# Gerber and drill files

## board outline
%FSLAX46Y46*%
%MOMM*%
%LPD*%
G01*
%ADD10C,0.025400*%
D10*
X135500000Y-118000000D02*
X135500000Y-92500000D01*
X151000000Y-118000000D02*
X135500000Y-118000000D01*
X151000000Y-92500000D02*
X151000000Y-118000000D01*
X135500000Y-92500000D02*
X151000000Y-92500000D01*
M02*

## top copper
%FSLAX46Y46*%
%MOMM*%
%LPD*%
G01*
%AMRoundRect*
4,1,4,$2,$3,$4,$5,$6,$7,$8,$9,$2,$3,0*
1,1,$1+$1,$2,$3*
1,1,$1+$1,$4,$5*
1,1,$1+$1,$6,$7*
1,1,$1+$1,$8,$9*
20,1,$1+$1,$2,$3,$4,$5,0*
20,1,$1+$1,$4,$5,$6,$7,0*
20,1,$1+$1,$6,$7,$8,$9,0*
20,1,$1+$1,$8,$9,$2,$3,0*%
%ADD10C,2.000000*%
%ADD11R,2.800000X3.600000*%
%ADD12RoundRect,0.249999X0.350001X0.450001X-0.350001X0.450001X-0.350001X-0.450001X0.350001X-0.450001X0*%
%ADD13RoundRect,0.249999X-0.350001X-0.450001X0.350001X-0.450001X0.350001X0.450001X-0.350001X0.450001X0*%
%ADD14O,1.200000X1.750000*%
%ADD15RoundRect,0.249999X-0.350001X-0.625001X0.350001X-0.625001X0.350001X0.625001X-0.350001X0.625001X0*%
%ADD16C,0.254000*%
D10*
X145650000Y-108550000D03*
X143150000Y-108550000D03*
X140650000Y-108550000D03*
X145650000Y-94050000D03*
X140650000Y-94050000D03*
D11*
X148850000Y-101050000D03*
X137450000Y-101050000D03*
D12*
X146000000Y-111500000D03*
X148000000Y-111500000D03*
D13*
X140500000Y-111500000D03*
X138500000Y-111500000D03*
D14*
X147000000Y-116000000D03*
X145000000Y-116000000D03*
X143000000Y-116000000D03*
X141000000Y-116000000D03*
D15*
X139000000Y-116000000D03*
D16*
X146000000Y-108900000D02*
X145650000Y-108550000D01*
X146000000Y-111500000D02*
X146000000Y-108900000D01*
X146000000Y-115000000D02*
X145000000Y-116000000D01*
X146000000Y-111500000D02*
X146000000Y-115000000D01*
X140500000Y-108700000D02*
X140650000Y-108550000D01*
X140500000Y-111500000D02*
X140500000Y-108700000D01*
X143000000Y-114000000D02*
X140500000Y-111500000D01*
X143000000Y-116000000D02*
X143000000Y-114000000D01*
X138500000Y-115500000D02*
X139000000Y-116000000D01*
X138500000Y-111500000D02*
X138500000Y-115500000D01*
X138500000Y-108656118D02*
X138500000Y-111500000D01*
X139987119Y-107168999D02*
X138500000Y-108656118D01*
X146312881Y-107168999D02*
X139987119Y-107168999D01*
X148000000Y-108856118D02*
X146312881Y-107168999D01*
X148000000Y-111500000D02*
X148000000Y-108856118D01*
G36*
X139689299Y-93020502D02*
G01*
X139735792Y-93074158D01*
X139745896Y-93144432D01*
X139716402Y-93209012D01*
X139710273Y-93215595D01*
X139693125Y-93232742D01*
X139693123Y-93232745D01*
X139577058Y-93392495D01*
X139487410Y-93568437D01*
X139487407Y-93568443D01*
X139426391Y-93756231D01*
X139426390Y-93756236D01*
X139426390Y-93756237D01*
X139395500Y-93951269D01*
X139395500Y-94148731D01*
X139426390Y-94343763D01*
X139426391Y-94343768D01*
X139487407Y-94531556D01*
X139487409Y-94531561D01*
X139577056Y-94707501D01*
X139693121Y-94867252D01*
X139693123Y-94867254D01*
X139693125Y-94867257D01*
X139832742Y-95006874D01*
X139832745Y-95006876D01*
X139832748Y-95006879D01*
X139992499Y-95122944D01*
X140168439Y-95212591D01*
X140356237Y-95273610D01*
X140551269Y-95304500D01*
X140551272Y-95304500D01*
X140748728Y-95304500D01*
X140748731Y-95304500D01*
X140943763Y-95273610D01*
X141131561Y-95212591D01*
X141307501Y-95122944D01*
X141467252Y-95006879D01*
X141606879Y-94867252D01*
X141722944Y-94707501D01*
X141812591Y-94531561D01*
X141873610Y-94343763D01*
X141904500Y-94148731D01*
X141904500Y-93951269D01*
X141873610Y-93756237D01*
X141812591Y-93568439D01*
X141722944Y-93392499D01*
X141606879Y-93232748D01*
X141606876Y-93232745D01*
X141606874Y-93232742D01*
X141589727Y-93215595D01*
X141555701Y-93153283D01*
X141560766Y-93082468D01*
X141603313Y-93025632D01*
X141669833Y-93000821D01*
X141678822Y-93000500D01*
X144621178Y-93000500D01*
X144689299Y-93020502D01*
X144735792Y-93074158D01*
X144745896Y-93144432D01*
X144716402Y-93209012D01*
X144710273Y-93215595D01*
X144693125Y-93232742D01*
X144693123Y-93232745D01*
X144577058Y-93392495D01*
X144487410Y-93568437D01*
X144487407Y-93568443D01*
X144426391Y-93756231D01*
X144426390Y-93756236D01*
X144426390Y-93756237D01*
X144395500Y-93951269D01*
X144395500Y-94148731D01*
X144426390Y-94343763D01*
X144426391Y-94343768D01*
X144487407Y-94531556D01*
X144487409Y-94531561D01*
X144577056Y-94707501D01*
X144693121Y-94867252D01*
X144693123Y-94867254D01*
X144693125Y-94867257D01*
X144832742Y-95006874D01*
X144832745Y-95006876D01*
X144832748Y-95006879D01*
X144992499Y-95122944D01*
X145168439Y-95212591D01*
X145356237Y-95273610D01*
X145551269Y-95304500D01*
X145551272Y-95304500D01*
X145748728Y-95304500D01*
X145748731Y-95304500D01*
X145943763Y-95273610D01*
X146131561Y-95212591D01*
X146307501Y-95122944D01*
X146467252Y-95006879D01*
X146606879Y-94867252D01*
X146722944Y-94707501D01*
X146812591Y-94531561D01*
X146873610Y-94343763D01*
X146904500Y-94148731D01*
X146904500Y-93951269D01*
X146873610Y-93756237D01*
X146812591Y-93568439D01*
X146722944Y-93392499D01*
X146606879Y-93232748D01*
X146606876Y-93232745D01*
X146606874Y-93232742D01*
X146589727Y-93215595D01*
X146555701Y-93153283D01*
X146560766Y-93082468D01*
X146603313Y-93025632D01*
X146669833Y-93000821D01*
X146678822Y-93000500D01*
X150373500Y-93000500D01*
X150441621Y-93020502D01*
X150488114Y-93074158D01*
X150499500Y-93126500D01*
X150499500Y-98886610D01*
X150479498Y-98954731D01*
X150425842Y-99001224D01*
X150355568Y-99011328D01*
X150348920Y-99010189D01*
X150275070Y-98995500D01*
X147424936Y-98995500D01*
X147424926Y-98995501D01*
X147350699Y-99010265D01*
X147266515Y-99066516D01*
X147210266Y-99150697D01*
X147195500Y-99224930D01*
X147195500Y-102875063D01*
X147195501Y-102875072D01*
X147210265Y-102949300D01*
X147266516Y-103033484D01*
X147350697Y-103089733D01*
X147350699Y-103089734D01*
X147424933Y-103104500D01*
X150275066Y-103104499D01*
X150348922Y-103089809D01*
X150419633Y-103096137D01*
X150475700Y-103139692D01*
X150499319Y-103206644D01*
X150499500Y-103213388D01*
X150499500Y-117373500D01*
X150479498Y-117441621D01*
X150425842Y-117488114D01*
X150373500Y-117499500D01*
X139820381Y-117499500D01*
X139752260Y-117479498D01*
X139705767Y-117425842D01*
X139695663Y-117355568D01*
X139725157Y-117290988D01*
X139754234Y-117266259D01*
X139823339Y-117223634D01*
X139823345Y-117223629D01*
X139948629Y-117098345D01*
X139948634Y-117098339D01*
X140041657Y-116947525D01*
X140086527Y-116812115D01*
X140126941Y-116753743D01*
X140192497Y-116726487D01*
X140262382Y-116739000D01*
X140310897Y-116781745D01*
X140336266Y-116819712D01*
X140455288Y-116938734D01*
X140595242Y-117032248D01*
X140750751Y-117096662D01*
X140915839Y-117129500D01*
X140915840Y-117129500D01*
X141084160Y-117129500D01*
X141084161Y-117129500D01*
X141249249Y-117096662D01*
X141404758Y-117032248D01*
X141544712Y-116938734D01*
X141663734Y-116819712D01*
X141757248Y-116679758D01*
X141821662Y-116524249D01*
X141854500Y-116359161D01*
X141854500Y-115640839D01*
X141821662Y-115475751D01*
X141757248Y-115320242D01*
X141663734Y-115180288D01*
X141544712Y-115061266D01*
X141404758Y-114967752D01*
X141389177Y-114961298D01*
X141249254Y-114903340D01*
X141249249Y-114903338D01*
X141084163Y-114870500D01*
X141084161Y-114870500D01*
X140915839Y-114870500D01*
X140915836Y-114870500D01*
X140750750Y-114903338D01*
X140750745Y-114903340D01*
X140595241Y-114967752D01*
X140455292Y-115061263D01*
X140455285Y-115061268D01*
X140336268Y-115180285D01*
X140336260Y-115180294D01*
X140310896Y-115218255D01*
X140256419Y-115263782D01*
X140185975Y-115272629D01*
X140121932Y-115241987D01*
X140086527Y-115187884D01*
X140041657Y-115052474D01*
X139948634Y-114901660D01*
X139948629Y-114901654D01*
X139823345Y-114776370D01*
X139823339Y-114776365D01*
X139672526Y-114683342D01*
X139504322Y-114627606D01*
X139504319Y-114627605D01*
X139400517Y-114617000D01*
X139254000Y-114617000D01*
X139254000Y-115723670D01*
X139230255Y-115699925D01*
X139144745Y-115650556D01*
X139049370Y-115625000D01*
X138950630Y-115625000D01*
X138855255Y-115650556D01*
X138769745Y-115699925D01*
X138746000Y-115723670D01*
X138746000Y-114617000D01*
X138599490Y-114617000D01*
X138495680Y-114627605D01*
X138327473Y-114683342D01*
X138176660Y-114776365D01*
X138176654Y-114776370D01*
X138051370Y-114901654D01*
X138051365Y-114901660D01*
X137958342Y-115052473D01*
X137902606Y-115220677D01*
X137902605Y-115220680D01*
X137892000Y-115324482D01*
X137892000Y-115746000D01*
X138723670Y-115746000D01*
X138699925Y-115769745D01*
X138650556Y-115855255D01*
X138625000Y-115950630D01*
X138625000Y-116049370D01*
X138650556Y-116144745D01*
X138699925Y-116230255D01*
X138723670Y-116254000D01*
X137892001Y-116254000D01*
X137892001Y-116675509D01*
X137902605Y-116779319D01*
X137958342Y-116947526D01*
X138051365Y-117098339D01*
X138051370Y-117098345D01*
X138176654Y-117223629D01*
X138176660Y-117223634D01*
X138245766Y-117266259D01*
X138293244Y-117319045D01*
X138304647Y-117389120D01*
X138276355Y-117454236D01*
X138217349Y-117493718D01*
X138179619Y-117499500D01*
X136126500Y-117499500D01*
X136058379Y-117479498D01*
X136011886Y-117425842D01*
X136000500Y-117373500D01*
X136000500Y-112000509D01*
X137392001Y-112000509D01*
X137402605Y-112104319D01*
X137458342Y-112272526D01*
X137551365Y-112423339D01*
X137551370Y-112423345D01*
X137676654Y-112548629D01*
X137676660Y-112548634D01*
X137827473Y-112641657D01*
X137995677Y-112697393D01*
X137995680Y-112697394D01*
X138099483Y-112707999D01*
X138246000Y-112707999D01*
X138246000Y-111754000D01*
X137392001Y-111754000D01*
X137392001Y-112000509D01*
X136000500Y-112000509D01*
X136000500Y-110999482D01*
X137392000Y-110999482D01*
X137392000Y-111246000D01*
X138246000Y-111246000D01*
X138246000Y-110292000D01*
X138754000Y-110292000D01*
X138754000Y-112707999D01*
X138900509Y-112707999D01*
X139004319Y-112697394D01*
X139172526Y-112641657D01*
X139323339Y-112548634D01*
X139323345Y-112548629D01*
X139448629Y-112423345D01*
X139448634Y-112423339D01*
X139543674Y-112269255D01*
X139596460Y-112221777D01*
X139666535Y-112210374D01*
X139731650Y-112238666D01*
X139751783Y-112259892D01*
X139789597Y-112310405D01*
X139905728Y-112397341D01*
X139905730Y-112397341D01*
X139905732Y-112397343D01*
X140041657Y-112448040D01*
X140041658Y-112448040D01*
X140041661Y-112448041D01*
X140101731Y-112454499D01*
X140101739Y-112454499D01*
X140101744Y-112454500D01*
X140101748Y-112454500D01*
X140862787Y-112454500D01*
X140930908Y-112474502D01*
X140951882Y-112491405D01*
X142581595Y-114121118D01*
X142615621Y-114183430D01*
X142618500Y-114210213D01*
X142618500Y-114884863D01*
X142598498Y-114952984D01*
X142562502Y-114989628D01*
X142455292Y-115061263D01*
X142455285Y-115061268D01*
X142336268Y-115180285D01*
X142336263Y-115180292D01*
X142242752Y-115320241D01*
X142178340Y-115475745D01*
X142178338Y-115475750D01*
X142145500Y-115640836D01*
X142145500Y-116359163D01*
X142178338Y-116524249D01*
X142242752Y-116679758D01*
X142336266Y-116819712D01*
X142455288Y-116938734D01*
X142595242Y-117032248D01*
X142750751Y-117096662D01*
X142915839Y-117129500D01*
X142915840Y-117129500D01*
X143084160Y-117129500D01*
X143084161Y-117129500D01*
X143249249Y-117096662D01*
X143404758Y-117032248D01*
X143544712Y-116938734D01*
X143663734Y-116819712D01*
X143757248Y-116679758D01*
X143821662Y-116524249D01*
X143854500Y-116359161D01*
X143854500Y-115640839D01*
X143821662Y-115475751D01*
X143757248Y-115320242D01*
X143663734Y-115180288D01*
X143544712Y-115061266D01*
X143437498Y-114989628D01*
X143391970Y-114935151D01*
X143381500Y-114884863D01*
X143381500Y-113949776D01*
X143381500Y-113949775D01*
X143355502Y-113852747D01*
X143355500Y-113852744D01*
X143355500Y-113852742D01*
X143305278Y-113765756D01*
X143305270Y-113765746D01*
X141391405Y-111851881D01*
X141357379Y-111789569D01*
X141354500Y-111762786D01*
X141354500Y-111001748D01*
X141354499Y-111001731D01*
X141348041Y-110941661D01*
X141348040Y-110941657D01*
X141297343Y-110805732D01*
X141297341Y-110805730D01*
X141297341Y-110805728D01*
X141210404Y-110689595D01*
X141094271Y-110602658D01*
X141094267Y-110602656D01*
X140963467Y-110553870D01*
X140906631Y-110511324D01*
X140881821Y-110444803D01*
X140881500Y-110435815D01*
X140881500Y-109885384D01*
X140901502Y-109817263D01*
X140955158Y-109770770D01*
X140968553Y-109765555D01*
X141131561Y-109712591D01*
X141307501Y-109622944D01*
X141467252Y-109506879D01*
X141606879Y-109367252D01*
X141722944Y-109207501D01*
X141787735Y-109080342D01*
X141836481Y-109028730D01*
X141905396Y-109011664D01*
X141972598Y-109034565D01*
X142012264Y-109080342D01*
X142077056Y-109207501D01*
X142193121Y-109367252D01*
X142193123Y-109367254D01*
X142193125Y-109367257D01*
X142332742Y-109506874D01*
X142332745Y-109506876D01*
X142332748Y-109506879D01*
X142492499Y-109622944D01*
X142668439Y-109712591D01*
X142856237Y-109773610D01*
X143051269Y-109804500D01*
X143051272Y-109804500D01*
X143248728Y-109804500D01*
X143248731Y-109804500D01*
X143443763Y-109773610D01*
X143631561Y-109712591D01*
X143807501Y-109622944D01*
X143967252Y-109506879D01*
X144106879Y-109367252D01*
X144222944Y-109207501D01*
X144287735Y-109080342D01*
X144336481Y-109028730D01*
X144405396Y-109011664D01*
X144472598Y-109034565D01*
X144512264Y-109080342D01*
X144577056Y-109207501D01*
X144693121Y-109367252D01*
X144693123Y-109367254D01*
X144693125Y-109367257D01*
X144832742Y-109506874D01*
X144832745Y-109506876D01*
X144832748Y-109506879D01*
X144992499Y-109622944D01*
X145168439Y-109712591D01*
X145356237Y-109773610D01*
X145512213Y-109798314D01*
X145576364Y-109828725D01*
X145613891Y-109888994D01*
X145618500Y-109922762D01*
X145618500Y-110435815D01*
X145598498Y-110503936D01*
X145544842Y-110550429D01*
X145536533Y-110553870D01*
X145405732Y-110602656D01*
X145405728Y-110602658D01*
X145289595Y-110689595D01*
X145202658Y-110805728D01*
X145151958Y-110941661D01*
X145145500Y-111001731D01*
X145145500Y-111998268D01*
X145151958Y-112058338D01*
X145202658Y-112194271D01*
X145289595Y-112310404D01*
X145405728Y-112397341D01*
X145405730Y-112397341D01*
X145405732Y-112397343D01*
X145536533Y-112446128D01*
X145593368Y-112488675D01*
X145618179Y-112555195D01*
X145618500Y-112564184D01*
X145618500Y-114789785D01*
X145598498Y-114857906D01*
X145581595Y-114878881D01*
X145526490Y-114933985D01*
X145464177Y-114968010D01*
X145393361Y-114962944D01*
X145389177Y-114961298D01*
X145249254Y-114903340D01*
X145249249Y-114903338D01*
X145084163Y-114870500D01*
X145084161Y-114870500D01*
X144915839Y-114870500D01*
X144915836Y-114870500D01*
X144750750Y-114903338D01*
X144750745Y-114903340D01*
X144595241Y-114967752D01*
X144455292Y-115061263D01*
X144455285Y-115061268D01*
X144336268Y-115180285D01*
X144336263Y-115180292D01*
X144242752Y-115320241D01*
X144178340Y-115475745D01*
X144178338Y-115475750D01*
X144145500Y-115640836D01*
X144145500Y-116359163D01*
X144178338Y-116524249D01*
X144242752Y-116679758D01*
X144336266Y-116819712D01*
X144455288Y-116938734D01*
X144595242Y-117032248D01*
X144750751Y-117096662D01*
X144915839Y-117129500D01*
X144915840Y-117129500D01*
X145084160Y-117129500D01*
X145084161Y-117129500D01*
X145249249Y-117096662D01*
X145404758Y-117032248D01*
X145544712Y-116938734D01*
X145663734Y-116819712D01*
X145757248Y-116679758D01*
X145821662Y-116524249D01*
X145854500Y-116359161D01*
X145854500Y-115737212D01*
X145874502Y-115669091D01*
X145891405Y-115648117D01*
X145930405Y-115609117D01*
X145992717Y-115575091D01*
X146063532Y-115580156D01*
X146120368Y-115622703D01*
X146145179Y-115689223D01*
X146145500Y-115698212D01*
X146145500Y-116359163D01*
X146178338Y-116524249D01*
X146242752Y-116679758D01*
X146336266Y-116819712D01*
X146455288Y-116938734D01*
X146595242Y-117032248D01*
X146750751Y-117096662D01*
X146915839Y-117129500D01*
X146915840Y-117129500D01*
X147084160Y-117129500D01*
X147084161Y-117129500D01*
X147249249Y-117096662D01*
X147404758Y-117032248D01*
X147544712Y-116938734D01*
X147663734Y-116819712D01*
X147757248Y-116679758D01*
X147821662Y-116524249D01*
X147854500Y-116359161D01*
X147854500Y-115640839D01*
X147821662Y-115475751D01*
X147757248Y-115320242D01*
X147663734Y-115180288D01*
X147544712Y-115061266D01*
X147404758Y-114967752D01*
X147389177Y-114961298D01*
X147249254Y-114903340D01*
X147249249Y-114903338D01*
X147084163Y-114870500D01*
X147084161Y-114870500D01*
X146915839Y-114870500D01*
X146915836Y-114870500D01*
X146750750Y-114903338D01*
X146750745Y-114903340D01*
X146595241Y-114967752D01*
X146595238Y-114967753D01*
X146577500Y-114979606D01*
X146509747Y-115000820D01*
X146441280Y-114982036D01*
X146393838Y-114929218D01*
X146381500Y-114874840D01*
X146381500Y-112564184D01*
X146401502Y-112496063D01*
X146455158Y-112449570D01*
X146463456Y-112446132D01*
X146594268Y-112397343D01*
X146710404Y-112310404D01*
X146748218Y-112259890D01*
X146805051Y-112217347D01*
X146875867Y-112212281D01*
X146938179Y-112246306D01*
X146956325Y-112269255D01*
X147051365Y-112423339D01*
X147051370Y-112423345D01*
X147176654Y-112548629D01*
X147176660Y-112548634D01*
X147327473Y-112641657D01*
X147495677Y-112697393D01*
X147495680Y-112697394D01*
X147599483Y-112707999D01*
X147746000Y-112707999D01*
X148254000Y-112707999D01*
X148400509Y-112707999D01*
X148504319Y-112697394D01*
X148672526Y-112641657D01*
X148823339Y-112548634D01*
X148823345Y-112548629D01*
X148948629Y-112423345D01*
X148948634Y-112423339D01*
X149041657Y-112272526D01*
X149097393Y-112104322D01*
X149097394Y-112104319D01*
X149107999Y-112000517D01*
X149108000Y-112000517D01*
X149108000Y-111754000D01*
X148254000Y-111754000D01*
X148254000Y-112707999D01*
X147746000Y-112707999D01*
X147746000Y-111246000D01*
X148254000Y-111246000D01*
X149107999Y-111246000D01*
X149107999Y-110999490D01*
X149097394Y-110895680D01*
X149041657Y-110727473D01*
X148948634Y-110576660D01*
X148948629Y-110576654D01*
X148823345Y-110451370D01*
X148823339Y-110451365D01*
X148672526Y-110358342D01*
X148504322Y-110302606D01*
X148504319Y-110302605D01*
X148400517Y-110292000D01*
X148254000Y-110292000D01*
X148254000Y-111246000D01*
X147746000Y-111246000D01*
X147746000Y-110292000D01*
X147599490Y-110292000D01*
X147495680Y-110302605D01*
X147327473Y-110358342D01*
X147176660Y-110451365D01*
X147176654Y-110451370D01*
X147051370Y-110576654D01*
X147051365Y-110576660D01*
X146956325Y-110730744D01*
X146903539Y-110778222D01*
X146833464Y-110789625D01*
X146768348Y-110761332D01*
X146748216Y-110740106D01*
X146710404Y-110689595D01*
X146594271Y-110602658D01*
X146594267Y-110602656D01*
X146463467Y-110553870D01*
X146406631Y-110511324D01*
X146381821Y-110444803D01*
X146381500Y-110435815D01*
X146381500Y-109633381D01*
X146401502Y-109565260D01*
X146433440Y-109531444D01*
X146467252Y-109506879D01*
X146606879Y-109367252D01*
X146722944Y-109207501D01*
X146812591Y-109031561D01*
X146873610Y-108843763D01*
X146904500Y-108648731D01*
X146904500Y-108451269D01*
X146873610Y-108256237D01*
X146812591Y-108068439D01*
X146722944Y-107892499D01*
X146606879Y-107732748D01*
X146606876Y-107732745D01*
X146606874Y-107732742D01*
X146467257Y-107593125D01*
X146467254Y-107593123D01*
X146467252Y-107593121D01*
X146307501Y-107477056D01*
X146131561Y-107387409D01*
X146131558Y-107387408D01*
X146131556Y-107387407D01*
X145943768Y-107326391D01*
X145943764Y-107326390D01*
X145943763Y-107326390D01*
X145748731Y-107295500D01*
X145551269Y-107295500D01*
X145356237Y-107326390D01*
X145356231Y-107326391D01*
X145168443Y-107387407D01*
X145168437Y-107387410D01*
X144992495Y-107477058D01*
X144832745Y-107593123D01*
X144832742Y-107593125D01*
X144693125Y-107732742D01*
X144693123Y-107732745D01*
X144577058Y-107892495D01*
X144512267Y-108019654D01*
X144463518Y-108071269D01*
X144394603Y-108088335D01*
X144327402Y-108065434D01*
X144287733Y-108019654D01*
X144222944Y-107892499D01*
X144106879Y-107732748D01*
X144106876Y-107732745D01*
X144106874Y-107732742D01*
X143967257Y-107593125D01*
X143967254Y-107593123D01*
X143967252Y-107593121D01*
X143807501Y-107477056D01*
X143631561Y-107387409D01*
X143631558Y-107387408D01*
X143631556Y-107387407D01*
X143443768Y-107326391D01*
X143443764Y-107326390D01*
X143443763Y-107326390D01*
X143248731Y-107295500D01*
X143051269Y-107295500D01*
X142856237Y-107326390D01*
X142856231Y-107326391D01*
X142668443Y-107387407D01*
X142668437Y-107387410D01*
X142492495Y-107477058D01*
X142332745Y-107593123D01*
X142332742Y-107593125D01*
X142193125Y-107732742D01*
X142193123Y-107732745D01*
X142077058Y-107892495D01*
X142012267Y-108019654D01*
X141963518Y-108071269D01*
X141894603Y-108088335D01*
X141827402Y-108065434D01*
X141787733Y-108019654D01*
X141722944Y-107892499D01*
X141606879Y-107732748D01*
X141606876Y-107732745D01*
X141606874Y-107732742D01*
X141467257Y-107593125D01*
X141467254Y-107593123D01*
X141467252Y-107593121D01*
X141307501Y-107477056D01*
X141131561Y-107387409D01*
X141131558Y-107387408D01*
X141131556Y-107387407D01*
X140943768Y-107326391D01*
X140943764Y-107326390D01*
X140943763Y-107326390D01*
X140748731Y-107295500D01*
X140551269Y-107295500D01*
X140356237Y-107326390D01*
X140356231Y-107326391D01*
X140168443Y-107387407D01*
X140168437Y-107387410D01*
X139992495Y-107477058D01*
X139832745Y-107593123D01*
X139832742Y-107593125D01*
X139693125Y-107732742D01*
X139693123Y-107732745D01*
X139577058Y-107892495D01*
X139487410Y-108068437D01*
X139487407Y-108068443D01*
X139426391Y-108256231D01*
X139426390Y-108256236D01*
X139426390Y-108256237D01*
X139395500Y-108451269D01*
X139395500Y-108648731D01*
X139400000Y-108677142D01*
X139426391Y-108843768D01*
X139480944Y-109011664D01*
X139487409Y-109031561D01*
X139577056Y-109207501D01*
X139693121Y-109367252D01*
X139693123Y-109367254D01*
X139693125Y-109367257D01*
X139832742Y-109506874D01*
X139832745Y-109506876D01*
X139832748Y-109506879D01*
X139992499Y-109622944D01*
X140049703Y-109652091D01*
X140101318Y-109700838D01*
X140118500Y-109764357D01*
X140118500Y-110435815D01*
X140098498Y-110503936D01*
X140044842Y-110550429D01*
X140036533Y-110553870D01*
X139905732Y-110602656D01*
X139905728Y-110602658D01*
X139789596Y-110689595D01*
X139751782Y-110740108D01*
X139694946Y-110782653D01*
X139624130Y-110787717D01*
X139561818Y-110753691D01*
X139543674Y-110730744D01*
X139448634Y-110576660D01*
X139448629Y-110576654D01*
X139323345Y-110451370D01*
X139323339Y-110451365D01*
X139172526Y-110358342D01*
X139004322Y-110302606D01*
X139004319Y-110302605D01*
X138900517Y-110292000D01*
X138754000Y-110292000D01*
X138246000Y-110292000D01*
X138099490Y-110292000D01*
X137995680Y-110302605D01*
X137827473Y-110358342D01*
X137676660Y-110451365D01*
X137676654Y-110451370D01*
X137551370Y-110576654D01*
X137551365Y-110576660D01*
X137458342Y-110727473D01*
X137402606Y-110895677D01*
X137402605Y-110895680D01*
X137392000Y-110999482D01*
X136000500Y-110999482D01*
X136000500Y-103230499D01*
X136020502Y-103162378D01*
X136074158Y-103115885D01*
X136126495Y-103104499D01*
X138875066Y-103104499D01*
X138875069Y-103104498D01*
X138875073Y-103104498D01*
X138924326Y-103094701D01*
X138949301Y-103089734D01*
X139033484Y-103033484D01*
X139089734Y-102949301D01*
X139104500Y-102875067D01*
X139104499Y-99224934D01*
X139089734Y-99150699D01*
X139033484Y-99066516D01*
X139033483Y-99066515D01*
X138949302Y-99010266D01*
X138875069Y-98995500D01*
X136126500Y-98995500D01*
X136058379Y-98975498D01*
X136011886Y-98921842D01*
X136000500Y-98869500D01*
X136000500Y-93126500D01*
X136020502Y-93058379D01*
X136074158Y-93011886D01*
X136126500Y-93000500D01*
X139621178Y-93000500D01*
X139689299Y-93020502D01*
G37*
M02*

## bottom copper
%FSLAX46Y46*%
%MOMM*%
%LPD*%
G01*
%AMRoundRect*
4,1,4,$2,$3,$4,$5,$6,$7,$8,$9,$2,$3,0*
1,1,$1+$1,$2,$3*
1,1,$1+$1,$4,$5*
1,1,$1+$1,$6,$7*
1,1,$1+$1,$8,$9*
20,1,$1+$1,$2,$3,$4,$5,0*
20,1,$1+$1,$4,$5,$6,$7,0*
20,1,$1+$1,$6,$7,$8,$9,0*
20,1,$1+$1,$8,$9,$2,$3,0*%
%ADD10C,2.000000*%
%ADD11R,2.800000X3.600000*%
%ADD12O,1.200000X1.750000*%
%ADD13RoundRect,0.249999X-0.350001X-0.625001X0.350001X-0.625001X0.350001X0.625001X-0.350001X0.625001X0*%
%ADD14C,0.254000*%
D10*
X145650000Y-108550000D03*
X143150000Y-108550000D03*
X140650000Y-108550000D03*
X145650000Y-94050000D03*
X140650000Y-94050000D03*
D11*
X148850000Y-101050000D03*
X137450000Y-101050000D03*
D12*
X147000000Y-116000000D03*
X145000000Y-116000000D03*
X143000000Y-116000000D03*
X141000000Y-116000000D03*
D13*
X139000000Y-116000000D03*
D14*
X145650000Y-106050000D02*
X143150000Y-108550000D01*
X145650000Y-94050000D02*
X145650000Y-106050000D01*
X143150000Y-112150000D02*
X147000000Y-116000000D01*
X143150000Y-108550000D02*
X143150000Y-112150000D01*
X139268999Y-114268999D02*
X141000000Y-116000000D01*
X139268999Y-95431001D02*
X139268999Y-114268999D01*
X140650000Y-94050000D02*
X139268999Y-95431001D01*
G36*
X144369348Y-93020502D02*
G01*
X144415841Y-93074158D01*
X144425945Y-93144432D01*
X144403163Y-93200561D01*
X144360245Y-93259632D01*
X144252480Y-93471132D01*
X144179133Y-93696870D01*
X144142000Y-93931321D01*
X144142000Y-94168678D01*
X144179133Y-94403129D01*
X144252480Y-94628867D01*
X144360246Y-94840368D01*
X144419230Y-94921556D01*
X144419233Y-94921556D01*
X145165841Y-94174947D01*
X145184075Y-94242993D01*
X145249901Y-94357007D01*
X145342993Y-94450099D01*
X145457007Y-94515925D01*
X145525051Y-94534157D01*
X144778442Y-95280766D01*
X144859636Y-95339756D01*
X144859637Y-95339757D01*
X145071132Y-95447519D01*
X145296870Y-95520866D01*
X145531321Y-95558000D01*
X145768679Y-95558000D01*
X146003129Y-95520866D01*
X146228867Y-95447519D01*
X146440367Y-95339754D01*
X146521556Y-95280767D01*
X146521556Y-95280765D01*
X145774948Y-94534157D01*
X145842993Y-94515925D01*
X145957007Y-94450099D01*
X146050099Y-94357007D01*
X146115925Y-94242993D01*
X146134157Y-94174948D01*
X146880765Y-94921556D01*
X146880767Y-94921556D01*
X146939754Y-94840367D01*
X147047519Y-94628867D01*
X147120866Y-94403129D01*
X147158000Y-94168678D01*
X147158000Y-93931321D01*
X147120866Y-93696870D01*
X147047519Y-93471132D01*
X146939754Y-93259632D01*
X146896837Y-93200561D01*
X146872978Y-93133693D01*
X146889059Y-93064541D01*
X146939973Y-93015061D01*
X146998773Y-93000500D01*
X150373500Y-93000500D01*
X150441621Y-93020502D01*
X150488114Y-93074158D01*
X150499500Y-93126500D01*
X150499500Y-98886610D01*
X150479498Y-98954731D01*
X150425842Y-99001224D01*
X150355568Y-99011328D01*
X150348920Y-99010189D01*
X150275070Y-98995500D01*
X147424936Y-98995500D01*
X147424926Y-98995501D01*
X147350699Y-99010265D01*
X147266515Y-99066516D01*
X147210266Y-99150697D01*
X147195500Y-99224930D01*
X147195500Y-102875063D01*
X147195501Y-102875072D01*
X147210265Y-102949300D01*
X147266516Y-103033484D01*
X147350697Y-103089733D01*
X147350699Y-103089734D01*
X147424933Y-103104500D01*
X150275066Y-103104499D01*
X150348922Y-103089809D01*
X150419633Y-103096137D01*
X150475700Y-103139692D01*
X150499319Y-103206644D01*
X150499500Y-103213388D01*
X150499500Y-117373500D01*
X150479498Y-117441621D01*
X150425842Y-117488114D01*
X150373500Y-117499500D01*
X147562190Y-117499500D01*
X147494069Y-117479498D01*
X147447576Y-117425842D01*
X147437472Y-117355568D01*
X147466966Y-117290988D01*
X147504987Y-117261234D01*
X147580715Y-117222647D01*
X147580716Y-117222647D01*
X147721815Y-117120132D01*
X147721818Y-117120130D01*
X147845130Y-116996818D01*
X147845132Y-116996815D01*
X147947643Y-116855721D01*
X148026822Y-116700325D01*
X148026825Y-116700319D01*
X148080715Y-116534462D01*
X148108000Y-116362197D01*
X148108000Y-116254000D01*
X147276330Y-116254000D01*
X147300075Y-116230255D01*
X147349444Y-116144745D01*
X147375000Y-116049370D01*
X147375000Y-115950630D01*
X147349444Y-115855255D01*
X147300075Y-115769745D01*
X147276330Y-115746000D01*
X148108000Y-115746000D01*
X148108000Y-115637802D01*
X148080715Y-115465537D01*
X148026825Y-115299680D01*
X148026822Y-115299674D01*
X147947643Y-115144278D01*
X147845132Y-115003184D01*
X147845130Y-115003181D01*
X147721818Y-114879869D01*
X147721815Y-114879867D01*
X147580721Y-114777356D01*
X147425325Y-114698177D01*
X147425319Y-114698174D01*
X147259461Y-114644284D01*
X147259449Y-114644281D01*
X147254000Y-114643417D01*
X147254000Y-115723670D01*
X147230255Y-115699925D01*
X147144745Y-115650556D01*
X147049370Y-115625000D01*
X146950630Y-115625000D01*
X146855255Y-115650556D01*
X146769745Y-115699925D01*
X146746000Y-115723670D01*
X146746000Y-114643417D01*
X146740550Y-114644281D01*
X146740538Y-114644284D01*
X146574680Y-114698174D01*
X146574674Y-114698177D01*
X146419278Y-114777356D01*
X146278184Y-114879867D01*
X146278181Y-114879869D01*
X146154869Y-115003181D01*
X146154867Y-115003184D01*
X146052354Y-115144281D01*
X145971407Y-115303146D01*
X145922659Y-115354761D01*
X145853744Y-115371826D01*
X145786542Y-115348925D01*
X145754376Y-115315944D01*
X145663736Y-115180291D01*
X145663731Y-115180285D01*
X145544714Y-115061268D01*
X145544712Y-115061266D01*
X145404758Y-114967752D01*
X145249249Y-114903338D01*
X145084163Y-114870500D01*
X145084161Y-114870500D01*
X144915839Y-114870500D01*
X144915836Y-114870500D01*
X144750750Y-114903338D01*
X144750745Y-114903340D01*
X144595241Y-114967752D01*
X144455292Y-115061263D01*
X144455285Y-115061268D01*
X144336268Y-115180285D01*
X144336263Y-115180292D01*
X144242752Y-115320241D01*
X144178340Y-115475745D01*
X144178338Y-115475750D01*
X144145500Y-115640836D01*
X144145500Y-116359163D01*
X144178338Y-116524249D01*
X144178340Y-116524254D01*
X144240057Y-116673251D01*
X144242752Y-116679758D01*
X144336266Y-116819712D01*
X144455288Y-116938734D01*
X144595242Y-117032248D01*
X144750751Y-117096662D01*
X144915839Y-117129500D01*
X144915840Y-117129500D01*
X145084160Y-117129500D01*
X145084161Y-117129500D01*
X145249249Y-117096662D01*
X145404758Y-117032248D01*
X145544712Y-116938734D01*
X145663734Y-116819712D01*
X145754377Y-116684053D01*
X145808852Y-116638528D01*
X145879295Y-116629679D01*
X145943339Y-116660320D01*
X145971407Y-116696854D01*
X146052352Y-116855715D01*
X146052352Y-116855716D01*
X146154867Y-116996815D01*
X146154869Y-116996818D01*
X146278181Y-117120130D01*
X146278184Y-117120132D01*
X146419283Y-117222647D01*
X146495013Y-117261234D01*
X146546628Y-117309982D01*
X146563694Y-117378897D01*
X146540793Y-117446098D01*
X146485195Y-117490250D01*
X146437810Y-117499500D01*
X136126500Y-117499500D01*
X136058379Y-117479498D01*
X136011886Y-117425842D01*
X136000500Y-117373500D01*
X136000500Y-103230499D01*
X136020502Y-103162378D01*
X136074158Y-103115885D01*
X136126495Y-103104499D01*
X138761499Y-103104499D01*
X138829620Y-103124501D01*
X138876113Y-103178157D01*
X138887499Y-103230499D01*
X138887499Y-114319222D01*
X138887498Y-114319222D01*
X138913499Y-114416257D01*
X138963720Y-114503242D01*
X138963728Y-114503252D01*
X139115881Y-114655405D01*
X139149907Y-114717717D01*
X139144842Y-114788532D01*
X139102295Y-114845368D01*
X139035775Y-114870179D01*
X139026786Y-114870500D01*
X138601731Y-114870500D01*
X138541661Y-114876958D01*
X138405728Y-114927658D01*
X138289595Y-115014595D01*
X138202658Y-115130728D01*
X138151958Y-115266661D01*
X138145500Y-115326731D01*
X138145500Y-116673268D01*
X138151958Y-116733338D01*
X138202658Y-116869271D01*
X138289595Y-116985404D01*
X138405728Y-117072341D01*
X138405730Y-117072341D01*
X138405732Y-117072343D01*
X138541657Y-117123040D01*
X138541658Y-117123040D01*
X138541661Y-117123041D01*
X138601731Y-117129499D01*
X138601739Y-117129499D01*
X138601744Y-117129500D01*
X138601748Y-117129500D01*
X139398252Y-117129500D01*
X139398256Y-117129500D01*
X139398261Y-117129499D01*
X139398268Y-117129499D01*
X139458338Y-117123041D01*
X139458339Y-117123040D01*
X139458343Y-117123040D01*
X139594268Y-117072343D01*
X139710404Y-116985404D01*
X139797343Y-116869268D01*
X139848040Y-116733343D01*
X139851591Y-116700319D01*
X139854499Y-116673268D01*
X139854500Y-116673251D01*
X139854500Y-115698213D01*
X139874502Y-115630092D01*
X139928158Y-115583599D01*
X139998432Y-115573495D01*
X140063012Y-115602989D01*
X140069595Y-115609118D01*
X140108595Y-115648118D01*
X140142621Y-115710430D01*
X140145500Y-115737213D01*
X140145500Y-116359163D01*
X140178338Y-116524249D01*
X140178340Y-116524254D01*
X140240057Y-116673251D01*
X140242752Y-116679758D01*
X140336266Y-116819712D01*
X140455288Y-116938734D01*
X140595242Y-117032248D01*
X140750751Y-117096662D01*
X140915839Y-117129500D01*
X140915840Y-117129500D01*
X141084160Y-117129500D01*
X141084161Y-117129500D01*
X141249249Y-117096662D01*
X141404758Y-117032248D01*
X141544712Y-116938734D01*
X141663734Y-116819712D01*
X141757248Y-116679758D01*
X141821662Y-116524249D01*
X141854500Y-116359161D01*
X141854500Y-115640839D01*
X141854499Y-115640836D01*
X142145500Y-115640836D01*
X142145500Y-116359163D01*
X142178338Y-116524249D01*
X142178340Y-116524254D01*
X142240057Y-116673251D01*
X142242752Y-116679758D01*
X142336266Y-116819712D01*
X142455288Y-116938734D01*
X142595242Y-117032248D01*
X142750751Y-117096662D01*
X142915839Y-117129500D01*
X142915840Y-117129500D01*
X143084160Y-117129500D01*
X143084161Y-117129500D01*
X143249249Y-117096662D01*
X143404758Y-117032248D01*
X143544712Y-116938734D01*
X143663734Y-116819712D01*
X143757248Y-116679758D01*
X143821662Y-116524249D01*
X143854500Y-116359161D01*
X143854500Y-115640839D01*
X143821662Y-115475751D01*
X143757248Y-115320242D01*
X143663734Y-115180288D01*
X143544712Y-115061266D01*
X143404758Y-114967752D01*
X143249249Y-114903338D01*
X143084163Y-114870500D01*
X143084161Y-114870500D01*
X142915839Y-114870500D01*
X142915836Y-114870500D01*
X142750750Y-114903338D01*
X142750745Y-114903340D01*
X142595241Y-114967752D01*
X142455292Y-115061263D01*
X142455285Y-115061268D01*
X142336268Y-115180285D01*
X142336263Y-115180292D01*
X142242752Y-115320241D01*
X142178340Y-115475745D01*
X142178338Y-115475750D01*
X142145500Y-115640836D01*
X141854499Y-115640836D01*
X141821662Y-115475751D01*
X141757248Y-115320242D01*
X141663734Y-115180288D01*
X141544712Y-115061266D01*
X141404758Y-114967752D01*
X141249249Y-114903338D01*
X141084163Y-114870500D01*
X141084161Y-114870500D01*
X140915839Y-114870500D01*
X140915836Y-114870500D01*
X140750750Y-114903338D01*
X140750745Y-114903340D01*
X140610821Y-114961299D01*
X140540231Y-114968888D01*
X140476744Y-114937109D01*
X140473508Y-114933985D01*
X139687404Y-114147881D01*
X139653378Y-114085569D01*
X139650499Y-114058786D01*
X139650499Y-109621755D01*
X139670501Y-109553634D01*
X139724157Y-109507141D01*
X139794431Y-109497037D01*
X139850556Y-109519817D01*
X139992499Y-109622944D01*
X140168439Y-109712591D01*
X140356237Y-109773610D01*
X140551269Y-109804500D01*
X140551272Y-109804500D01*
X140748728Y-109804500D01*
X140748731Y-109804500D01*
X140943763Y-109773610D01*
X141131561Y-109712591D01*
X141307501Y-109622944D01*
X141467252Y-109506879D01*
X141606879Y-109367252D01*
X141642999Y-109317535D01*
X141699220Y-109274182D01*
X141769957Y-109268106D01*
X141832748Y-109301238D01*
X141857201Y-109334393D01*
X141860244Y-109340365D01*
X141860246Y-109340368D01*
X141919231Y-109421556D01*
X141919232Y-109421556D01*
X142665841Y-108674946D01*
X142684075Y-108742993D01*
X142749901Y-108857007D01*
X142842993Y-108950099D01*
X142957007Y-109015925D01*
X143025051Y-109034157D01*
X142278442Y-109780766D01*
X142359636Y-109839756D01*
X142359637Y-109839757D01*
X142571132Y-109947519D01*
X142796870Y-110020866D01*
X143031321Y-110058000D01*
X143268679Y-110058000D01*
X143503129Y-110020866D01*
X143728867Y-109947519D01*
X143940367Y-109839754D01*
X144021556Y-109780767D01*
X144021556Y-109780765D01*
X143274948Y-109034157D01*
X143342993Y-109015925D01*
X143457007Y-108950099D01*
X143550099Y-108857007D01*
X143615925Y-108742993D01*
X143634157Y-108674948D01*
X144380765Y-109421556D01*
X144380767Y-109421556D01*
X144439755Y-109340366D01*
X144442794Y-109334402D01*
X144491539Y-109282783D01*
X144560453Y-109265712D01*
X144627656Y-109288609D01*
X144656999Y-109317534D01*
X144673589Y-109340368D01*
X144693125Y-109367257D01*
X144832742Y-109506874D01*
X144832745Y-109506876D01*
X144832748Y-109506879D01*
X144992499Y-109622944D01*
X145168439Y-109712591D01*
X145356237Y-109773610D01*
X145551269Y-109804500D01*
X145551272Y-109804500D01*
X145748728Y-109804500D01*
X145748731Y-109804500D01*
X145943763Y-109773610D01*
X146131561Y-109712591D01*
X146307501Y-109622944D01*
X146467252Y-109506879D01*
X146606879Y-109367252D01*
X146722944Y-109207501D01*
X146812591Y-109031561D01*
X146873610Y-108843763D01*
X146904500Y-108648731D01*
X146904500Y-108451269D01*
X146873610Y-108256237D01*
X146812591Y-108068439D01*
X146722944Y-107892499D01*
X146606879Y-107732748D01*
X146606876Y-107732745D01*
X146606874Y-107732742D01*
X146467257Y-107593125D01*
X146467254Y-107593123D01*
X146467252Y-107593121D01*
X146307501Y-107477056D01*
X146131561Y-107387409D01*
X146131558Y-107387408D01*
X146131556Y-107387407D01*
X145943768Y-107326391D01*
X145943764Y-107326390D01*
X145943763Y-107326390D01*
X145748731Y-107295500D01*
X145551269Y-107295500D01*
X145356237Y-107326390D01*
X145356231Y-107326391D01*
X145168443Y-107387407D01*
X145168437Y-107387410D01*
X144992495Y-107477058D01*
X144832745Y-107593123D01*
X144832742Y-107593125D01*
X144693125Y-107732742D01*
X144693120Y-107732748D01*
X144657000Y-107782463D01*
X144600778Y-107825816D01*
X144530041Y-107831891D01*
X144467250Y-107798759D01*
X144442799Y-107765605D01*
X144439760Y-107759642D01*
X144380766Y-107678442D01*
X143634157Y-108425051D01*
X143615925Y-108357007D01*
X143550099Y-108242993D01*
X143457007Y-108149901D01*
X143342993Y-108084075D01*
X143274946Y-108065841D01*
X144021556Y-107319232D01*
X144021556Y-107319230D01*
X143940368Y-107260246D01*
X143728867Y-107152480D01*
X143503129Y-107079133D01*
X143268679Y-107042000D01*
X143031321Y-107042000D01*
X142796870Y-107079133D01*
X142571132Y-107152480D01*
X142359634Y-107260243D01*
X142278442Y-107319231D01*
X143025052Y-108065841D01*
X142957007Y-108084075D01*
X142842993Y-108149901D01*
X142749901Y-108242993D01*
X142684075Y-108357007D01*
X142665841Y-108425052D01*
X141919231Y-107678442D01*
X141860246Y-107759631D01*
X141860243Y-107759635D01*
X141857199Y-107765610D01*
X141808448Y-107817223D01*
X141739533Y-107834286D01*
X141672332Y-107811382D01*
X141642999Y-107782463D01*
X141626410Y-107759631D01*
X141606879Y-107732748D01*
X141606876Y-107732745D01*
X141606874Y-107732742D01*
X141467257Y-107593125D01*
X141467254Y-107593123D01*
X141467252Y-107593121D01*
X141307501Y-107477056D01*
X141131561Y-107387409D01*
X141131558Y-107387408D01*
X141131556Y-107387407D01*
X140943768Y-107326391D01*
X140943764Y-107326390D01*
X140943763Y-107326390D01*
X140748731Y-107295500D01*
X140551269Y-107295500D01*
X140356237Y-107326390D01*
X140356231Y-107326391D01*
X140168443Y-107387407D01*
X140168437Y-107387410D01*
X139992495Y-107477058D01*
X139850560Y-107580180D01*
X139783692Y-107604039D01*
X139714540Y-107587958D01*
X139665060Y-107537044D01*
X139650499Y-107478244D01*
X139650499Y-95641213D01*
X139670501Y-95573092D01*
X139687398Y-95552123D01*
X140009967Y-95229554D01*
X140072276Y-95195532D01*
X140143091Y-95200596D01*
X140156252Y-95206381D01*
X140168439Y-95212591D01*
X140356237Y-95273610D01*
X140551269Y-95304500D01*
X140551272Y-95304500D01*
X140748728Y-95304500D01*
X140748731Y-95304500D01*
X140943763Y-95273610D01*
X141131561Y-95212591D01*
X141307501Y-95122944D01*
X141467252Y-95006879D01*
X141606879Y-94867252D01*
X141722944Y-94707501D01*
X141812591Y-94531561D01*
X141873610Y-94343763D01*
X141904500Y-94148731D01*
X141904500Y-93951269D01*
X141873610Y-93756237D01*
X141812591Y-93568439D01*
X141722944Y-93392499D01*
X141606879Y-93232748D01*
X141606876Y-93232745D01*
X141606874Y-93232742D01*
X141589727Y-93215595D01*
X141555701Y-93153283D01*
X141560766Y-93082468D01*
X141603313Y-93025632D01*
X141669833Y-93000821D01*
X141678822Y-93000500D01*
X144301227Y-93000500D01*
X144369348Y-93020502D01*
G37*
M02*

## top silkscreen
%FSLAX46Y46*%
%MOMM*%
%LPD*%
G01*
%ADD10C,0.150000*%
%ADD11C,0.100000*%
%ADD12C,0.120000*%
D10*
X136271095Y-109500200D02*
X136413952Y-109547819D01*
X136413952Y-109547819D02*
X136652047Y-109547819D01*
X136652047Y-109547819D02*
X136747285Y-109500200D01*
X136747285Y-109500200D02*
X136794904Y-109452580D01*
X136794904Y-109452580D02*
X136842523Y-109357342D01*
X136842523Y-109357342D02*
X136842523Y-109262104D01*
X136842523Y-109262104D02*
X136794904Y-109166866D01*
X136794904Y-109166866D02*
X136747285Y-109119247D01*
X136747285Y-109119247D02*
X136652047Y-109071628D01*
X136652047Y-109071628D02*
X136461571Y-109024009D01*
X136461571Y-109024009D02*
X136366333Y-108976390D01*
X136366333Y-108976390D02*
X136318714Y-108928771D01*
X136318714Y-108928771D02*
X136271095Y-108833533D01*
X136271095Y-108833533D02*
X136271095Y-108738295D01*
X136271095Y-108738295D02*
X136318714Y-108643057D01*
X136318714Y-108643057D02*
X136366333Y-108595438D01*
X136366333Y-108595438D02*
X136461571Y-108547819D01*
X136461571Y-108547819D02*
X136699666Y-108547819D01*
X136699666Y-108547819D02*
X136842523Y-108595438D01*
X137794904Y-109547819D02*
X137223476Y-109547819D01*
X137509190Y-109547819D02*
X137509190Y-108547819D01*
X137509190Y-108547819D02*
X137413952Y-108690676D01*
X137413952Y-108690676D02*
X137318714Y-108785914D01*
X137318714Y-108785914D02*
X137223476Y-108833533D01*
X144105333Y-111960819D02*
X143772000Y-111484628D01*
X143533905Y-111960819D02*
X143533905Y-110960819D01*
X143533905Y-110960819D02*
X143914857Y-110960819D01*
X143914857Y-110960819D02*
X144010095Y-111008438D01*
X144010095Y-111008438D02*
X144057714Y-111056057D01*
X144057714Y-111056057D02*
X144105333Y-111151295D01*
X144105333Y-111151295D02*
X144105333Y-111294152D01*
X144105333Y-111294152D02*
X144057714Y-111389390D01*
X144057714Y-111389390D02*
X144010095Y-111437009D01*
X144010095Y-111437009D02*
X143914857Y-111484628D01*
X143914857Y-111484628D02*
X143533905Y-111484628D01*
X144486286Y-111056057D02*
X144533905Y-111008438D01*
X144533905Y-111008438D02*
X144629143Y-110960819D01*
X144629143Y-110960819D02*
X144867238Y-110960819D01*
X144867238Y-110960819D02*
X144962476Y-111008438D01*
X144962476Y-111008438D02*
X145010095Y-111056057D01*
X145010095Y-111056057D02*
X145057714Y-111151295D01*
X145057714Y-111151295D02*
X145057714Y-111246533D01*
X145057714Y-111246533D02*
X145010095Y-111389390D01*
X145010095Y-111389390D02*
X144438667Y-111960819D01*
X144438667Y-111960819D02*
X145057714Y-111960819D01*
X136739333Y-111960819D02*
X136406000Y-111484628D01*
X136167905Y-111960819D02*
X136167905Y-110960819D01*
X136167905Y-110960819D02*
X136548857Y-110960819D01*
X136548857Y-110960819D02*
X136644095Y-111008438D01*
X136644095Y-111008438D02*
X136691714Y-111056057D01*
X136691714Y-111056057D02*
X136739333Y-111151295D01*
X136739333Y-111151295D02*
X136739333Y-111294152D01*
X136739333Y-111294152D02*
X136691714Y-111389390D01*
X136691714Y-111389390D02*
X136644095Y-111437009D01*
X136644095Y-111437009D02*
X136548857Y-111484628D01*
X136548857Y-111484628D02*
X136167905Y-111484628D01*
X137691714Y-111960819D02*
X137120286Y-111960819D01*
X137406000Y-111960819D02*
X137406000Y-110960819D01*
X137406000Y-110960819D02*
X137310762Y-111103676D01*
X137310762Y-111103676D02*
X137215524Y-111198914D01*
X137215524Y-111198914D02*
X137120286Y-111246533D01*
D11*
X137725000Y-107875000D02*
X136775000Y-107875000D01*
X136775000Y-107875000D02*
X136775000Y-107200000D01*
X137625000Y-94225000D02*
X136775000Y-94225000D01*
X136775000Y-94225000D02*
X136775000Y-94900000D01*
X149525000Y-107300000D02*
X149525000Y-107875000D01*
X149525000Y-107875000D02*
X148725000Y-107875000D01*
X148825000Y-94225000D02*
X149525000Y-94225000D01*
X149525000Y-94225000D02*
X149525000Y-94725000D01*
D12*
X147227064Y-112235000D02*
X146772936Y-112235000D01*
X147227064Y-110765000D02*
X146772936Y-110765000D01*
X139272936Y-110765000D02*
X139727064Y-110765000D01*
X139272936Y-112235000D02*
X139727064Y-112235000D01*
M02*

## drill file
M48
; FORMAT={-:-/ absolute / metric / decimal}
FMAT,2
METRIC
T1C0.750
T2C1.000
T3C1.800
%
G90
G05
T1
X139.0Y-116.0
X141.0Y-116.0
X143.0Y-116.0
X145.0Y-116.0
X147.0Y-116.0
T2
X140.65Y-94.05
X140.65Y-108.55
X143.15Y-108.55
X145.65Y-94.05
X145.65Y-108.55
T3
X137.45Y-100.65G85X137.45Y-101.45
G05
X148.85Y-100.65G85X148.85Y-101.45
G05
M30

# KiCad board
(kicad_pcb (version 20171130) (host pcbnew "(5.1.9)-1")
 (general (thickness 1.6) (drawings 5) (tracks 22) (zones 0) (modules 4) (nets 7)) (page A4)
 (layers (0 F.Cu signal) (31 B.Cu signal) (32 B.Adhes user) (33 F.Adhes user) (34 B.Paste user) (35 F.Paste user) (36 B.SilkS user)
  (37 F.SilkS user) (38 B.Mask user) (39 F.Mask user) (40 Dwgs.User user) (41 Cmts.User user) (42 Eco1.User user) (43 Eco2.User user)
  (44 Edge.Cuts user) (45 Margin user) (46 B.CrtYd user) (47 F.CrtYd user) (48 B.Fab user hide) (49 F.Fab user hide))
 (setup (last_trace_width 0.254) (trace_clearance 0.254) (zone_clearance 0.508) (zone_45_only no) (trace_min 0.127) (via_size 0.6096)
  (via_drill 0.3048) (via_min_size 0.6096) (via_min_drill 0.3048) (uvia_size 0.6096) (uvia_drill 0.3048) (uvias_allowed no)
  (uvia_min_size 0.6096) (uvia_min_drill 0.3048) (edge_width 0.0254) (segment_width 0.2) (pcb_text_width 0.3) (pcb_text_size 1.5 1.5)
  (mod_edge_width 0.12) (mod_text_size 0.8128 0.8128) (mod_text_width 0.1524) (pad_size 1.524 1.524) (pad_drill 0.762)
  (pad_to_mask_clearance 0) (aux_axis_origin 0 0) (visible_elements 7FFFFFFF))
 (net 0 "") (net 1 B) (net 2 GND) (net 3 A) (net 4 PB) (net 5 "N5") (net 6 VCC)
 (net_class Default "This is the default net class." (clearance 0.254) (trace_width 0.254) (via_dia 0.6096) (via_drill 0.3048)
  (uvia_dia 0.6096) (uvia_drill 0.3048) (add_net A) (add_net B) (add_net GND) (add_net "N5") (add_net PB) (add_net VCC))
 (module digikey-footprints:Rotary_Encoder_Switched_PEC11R (layer F.Cu) (at 137.45 101.05)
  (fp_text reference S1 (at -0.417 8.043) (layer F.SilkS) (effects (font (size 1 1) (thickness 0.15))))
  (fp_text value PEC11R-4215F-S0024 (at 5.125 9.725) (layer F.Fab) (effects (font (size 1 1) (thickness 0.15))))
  (fp_line (start 0.275 6.825) (end -0.675 6.825) (layer F.SilkS) (width 0.1))
  (fp_line (start -0.675 6.825) (end -0.675 6.15) (layer F.SilkS) (width 0.1))
  (fp_line (start 0.175 -6.825) (end -0.675 -6.825) (layer F.SilkS) (width 0.1))
  (fp_line (start -0.675 -6.825) (end -0.675 -6.15) (layer F.SilkS) (width 0.1))
  (fp_line (start 12.075 6.25) (end 12.075 6.825) (layer F.SilkS) (width 0.1))
  (fp_line (start 12.075 6.825) (end 11.275 6.825) (layer F.SilkS) (width 0.1))
  (fp_line (start 11.375 -6.825) (end 12.075 -6.825) (layer F.SilkS) (width 0.1))
  (fp_line (start 12.075 -6.825) (end 12.075 -6.325) (layer F.SilkS) (width 0.1))
  (pad B thru_hole circle (at 8.2 7.5) (size 2 2) (drill 1) (layers *.Cu *.Mask) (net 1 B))
  (pad C thru_hole circle (at 5.7 7.5) (size 2 2) (drill 1) (layers *.Cu *.Mask) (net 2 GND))
  (pad A thru_hole circle (at 3.2 7.5) (size 2 2) (drill 1) (layers *.Cu *.Mask) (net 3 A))
  (pad 2 thru_hole circle (at 8.2 -7) (size 2 2) (drill 1) (layers *.Cu *.Mask) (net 2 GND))
  (pad 1 thru_hole circle (at 3.2 -7) (size 2 2) (drill 1) (layers *.Cu *.Mask) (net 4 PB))
  (pad 3 thru_hole rect (at 11.4 0) (size 2.8 3.6) (drill oval 1.8 2.6) (layers *.Cu *.Mask) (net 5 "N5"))
  (pad 3 thru_hole rect (at 0 0) (size 2.8 3.6) (drill oval 1.8 2.6) (layers *.Cu *.Mask) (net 5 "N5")))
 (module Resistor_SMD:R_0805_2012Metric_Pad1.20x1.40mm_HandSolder (layer F.Cu) (at 147 111.5 180)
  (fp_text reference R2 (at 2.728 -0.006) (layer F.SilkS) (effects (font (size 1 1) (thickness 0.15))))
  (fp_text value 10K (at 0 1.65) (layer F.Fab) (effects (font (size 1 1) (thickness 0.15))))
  (fp_line (start -0.227064 -0.735) (end 0.227064 -0.735) (layer F.SilkS) (width 0.12))
  (fp_line (start -0.227064 0.735) (end 0.227064 0.735) (layer F.SilkS) (width 0.12))
  (pad 2 smd roundrect (at 1 0 180) (size 1.2 1.4) (layers F.Cu F.Paste F.Mask) (roundrect_rratio 0.2083325) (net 1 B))
  (pad 1 smd roundrect (at -1 0 180) (size 1.2 1.4) (layers F.Cu F.Paste F.Mask) (roundrect_rratio 0.2083325) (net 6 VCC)))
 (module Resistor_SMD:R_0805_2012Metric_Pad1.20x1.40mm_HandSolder (layer F.Cu) (at 139.5 111.5)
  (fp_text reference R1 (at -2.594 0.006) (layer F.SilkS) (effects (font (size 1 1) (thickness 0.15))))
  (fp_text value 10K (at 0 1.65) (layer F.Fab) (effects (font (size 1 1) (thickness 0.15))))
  (fp_line (start -0.227064 -0.735) (end 0.227064 -0.735) (layer F.SilkS) (width 0.12))
  (fp_line (start -0.227064 0.735) (end 0.227064 0.735) (layer F.SilkS) (width 0.12))
  (pad 2 smd roundrect (at 1 0) (size 1.2 1.4) (layers F.Cu F.Paste F.Mask) (roundrect_rratio 0.2083325) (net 3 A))
  (pad 1 smd roundrect (at -1 0) (size 1.2 1.4) (layers F.Cu F.Paste F.Mask) (roundrect_rratio 0.2083325) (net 6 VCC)))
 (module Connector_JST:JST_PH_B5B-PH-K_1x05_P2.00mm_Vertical (layer B.Cu) (at 139 116)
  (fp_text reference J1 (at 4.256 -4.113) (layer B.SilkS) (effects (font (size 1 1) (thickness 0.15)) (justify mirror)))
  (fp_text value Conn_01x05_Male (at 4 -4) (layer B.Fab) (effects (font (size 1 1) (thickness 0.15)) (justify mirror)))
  (pad 5 thru_hole oval (at 8 0) (size 1.2 1.75) (drill 0.75) (layers *.Cu *.Mask) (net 2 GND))
  (pad 4 thru_hole oval (at 6 0) (size 1.2 1.75) (drill 0.75) (layers *.Cu *.Mask) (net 1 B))
  (pad 3 thru_hole oval (at 4 0) (size 1.2 1.75) (drill 0.75) (layers *.Cu *.Mask) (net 3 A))
  (pad 2 thru_hole oval (at 2 0) (size 1.2 1.75) (drill 0.75) (layers *.Cu *.Mask) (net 4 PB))
  (pad 1 thru_hole roundrect (at 0 0) (size 1.2 1.75) (drill 0.75) (layers *.Cu *.Mask) (roundrect_rratio 0.2083325) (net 6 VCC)))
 (gr_line (start 135.5 118) (end 135.5 92.5) (layer Edge.Cuts) (width 0.0254))
 (gr_line (start 151 118) (end 135.5 118) (layer Edge.Cuts) (width 0.0254))
 (gr_line (start 151 92.5) (end 151 118) (layer Edge.Cuts) (width 0.0254))
 (gr_line (start 135.5 92.5) (end 151 92.5) (layer Edge.Cuts) (width 0.0254))
 (segment (start 145.65 106.05) (end 143.15 108.55) (width 0.254) (layer B.Cu) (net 2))
 (segment (start 145.65 94.05) (end 145.65 106.05) (width 0.254) (layer B.Cu) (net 2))
 (segment (start 143.15 112.15) (end 147 116) (width 0.254) (layer B.Cu) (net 2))
 (segment (start 143.15 108.55) (end 143.15 112.15) (width 0.254) (layer B.Cu) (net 2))
 (segment (start 146 108.9) (end 145.65 108.55) (width 0.254) (layer F.Cu) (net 1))
 (segment (start 146 111.5) (end 146 108.9) (width 0.254) (layer F.Cu) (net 1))
 (segment (start 146 115) (end 145 116) (width 0.254) (layer F.Cu) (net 1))
 (segment (start 146 111.5) (end 146 115) (width 0.254) (layer F.Cu) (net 1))
 (segment (start 140.5 108.7) (end 140.65 108.55) (width 0.254) (layer F.Cu) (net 3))
 (segment (start 140.5 111.5) (end 140.5 108.7) (width 0.254) (layer F.Cu) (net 3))
 (segment (start 143 114) (end 140.5 111.5) (width 0.254) (layer F.Cu) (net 3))
 (segment (start 143 116) (end 143 114) (width 0.254) (layer F.Cu) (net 3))
 (segment (start 139.268999 114.268999) (end 141 116) (width 0.254) (layer B.Cu) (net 4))
 (segment (start 139.268999 95.431001) (end 139.268999 114.268999) (width 0.254) (layer B.Cu) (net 4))
 (segment (start 140.65 94.05) (end 139.268999 95.431001) (width 0.254) (layer B.Cu) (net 4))
 (segment (start 138.5 115.5) (end 139 116) (width 0.254) (layer F.Cu) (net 6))
 (segment (start 138.5 111.5) (end 138.5 115.5) (width 0.254) (layer F.Cu) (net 6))
 (segment (start 138.5 108.656118) (end 138.5 111.5) (width 0.254) (layer F.Cu) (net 6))
 (segment (start 139.987119 107.168999) (end 138.5 108.656118) (width 0.254) (layer F.Cu) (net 6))
 (segment (start 146.312881 107.168999) (end 139.987119 107.168999) (width 0.254) (layer F.Cu) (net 6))
 (segment (start 148 108.856118) (end 146.312881 107.168999) (width 0.254) (layer F.Cu) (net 6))
 (segment (start 148 111.5) (end 148 108.856118) (width 0.254) (layer F.Cu) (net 6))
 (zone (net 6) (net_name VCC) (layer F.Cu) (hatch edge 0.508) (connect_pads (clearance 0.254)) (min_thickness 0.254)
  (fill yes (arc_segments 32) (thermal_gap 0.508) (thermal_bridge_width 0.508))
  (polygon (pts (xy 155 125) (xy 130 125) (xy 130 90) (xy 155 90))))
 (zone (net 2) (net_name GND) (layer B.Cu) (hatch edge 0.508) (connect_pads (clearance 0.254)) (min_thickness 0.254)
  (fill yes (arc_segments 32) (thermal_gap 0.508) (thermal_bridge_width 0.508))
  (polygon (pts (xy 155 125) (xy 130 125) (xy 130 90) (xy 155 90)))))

